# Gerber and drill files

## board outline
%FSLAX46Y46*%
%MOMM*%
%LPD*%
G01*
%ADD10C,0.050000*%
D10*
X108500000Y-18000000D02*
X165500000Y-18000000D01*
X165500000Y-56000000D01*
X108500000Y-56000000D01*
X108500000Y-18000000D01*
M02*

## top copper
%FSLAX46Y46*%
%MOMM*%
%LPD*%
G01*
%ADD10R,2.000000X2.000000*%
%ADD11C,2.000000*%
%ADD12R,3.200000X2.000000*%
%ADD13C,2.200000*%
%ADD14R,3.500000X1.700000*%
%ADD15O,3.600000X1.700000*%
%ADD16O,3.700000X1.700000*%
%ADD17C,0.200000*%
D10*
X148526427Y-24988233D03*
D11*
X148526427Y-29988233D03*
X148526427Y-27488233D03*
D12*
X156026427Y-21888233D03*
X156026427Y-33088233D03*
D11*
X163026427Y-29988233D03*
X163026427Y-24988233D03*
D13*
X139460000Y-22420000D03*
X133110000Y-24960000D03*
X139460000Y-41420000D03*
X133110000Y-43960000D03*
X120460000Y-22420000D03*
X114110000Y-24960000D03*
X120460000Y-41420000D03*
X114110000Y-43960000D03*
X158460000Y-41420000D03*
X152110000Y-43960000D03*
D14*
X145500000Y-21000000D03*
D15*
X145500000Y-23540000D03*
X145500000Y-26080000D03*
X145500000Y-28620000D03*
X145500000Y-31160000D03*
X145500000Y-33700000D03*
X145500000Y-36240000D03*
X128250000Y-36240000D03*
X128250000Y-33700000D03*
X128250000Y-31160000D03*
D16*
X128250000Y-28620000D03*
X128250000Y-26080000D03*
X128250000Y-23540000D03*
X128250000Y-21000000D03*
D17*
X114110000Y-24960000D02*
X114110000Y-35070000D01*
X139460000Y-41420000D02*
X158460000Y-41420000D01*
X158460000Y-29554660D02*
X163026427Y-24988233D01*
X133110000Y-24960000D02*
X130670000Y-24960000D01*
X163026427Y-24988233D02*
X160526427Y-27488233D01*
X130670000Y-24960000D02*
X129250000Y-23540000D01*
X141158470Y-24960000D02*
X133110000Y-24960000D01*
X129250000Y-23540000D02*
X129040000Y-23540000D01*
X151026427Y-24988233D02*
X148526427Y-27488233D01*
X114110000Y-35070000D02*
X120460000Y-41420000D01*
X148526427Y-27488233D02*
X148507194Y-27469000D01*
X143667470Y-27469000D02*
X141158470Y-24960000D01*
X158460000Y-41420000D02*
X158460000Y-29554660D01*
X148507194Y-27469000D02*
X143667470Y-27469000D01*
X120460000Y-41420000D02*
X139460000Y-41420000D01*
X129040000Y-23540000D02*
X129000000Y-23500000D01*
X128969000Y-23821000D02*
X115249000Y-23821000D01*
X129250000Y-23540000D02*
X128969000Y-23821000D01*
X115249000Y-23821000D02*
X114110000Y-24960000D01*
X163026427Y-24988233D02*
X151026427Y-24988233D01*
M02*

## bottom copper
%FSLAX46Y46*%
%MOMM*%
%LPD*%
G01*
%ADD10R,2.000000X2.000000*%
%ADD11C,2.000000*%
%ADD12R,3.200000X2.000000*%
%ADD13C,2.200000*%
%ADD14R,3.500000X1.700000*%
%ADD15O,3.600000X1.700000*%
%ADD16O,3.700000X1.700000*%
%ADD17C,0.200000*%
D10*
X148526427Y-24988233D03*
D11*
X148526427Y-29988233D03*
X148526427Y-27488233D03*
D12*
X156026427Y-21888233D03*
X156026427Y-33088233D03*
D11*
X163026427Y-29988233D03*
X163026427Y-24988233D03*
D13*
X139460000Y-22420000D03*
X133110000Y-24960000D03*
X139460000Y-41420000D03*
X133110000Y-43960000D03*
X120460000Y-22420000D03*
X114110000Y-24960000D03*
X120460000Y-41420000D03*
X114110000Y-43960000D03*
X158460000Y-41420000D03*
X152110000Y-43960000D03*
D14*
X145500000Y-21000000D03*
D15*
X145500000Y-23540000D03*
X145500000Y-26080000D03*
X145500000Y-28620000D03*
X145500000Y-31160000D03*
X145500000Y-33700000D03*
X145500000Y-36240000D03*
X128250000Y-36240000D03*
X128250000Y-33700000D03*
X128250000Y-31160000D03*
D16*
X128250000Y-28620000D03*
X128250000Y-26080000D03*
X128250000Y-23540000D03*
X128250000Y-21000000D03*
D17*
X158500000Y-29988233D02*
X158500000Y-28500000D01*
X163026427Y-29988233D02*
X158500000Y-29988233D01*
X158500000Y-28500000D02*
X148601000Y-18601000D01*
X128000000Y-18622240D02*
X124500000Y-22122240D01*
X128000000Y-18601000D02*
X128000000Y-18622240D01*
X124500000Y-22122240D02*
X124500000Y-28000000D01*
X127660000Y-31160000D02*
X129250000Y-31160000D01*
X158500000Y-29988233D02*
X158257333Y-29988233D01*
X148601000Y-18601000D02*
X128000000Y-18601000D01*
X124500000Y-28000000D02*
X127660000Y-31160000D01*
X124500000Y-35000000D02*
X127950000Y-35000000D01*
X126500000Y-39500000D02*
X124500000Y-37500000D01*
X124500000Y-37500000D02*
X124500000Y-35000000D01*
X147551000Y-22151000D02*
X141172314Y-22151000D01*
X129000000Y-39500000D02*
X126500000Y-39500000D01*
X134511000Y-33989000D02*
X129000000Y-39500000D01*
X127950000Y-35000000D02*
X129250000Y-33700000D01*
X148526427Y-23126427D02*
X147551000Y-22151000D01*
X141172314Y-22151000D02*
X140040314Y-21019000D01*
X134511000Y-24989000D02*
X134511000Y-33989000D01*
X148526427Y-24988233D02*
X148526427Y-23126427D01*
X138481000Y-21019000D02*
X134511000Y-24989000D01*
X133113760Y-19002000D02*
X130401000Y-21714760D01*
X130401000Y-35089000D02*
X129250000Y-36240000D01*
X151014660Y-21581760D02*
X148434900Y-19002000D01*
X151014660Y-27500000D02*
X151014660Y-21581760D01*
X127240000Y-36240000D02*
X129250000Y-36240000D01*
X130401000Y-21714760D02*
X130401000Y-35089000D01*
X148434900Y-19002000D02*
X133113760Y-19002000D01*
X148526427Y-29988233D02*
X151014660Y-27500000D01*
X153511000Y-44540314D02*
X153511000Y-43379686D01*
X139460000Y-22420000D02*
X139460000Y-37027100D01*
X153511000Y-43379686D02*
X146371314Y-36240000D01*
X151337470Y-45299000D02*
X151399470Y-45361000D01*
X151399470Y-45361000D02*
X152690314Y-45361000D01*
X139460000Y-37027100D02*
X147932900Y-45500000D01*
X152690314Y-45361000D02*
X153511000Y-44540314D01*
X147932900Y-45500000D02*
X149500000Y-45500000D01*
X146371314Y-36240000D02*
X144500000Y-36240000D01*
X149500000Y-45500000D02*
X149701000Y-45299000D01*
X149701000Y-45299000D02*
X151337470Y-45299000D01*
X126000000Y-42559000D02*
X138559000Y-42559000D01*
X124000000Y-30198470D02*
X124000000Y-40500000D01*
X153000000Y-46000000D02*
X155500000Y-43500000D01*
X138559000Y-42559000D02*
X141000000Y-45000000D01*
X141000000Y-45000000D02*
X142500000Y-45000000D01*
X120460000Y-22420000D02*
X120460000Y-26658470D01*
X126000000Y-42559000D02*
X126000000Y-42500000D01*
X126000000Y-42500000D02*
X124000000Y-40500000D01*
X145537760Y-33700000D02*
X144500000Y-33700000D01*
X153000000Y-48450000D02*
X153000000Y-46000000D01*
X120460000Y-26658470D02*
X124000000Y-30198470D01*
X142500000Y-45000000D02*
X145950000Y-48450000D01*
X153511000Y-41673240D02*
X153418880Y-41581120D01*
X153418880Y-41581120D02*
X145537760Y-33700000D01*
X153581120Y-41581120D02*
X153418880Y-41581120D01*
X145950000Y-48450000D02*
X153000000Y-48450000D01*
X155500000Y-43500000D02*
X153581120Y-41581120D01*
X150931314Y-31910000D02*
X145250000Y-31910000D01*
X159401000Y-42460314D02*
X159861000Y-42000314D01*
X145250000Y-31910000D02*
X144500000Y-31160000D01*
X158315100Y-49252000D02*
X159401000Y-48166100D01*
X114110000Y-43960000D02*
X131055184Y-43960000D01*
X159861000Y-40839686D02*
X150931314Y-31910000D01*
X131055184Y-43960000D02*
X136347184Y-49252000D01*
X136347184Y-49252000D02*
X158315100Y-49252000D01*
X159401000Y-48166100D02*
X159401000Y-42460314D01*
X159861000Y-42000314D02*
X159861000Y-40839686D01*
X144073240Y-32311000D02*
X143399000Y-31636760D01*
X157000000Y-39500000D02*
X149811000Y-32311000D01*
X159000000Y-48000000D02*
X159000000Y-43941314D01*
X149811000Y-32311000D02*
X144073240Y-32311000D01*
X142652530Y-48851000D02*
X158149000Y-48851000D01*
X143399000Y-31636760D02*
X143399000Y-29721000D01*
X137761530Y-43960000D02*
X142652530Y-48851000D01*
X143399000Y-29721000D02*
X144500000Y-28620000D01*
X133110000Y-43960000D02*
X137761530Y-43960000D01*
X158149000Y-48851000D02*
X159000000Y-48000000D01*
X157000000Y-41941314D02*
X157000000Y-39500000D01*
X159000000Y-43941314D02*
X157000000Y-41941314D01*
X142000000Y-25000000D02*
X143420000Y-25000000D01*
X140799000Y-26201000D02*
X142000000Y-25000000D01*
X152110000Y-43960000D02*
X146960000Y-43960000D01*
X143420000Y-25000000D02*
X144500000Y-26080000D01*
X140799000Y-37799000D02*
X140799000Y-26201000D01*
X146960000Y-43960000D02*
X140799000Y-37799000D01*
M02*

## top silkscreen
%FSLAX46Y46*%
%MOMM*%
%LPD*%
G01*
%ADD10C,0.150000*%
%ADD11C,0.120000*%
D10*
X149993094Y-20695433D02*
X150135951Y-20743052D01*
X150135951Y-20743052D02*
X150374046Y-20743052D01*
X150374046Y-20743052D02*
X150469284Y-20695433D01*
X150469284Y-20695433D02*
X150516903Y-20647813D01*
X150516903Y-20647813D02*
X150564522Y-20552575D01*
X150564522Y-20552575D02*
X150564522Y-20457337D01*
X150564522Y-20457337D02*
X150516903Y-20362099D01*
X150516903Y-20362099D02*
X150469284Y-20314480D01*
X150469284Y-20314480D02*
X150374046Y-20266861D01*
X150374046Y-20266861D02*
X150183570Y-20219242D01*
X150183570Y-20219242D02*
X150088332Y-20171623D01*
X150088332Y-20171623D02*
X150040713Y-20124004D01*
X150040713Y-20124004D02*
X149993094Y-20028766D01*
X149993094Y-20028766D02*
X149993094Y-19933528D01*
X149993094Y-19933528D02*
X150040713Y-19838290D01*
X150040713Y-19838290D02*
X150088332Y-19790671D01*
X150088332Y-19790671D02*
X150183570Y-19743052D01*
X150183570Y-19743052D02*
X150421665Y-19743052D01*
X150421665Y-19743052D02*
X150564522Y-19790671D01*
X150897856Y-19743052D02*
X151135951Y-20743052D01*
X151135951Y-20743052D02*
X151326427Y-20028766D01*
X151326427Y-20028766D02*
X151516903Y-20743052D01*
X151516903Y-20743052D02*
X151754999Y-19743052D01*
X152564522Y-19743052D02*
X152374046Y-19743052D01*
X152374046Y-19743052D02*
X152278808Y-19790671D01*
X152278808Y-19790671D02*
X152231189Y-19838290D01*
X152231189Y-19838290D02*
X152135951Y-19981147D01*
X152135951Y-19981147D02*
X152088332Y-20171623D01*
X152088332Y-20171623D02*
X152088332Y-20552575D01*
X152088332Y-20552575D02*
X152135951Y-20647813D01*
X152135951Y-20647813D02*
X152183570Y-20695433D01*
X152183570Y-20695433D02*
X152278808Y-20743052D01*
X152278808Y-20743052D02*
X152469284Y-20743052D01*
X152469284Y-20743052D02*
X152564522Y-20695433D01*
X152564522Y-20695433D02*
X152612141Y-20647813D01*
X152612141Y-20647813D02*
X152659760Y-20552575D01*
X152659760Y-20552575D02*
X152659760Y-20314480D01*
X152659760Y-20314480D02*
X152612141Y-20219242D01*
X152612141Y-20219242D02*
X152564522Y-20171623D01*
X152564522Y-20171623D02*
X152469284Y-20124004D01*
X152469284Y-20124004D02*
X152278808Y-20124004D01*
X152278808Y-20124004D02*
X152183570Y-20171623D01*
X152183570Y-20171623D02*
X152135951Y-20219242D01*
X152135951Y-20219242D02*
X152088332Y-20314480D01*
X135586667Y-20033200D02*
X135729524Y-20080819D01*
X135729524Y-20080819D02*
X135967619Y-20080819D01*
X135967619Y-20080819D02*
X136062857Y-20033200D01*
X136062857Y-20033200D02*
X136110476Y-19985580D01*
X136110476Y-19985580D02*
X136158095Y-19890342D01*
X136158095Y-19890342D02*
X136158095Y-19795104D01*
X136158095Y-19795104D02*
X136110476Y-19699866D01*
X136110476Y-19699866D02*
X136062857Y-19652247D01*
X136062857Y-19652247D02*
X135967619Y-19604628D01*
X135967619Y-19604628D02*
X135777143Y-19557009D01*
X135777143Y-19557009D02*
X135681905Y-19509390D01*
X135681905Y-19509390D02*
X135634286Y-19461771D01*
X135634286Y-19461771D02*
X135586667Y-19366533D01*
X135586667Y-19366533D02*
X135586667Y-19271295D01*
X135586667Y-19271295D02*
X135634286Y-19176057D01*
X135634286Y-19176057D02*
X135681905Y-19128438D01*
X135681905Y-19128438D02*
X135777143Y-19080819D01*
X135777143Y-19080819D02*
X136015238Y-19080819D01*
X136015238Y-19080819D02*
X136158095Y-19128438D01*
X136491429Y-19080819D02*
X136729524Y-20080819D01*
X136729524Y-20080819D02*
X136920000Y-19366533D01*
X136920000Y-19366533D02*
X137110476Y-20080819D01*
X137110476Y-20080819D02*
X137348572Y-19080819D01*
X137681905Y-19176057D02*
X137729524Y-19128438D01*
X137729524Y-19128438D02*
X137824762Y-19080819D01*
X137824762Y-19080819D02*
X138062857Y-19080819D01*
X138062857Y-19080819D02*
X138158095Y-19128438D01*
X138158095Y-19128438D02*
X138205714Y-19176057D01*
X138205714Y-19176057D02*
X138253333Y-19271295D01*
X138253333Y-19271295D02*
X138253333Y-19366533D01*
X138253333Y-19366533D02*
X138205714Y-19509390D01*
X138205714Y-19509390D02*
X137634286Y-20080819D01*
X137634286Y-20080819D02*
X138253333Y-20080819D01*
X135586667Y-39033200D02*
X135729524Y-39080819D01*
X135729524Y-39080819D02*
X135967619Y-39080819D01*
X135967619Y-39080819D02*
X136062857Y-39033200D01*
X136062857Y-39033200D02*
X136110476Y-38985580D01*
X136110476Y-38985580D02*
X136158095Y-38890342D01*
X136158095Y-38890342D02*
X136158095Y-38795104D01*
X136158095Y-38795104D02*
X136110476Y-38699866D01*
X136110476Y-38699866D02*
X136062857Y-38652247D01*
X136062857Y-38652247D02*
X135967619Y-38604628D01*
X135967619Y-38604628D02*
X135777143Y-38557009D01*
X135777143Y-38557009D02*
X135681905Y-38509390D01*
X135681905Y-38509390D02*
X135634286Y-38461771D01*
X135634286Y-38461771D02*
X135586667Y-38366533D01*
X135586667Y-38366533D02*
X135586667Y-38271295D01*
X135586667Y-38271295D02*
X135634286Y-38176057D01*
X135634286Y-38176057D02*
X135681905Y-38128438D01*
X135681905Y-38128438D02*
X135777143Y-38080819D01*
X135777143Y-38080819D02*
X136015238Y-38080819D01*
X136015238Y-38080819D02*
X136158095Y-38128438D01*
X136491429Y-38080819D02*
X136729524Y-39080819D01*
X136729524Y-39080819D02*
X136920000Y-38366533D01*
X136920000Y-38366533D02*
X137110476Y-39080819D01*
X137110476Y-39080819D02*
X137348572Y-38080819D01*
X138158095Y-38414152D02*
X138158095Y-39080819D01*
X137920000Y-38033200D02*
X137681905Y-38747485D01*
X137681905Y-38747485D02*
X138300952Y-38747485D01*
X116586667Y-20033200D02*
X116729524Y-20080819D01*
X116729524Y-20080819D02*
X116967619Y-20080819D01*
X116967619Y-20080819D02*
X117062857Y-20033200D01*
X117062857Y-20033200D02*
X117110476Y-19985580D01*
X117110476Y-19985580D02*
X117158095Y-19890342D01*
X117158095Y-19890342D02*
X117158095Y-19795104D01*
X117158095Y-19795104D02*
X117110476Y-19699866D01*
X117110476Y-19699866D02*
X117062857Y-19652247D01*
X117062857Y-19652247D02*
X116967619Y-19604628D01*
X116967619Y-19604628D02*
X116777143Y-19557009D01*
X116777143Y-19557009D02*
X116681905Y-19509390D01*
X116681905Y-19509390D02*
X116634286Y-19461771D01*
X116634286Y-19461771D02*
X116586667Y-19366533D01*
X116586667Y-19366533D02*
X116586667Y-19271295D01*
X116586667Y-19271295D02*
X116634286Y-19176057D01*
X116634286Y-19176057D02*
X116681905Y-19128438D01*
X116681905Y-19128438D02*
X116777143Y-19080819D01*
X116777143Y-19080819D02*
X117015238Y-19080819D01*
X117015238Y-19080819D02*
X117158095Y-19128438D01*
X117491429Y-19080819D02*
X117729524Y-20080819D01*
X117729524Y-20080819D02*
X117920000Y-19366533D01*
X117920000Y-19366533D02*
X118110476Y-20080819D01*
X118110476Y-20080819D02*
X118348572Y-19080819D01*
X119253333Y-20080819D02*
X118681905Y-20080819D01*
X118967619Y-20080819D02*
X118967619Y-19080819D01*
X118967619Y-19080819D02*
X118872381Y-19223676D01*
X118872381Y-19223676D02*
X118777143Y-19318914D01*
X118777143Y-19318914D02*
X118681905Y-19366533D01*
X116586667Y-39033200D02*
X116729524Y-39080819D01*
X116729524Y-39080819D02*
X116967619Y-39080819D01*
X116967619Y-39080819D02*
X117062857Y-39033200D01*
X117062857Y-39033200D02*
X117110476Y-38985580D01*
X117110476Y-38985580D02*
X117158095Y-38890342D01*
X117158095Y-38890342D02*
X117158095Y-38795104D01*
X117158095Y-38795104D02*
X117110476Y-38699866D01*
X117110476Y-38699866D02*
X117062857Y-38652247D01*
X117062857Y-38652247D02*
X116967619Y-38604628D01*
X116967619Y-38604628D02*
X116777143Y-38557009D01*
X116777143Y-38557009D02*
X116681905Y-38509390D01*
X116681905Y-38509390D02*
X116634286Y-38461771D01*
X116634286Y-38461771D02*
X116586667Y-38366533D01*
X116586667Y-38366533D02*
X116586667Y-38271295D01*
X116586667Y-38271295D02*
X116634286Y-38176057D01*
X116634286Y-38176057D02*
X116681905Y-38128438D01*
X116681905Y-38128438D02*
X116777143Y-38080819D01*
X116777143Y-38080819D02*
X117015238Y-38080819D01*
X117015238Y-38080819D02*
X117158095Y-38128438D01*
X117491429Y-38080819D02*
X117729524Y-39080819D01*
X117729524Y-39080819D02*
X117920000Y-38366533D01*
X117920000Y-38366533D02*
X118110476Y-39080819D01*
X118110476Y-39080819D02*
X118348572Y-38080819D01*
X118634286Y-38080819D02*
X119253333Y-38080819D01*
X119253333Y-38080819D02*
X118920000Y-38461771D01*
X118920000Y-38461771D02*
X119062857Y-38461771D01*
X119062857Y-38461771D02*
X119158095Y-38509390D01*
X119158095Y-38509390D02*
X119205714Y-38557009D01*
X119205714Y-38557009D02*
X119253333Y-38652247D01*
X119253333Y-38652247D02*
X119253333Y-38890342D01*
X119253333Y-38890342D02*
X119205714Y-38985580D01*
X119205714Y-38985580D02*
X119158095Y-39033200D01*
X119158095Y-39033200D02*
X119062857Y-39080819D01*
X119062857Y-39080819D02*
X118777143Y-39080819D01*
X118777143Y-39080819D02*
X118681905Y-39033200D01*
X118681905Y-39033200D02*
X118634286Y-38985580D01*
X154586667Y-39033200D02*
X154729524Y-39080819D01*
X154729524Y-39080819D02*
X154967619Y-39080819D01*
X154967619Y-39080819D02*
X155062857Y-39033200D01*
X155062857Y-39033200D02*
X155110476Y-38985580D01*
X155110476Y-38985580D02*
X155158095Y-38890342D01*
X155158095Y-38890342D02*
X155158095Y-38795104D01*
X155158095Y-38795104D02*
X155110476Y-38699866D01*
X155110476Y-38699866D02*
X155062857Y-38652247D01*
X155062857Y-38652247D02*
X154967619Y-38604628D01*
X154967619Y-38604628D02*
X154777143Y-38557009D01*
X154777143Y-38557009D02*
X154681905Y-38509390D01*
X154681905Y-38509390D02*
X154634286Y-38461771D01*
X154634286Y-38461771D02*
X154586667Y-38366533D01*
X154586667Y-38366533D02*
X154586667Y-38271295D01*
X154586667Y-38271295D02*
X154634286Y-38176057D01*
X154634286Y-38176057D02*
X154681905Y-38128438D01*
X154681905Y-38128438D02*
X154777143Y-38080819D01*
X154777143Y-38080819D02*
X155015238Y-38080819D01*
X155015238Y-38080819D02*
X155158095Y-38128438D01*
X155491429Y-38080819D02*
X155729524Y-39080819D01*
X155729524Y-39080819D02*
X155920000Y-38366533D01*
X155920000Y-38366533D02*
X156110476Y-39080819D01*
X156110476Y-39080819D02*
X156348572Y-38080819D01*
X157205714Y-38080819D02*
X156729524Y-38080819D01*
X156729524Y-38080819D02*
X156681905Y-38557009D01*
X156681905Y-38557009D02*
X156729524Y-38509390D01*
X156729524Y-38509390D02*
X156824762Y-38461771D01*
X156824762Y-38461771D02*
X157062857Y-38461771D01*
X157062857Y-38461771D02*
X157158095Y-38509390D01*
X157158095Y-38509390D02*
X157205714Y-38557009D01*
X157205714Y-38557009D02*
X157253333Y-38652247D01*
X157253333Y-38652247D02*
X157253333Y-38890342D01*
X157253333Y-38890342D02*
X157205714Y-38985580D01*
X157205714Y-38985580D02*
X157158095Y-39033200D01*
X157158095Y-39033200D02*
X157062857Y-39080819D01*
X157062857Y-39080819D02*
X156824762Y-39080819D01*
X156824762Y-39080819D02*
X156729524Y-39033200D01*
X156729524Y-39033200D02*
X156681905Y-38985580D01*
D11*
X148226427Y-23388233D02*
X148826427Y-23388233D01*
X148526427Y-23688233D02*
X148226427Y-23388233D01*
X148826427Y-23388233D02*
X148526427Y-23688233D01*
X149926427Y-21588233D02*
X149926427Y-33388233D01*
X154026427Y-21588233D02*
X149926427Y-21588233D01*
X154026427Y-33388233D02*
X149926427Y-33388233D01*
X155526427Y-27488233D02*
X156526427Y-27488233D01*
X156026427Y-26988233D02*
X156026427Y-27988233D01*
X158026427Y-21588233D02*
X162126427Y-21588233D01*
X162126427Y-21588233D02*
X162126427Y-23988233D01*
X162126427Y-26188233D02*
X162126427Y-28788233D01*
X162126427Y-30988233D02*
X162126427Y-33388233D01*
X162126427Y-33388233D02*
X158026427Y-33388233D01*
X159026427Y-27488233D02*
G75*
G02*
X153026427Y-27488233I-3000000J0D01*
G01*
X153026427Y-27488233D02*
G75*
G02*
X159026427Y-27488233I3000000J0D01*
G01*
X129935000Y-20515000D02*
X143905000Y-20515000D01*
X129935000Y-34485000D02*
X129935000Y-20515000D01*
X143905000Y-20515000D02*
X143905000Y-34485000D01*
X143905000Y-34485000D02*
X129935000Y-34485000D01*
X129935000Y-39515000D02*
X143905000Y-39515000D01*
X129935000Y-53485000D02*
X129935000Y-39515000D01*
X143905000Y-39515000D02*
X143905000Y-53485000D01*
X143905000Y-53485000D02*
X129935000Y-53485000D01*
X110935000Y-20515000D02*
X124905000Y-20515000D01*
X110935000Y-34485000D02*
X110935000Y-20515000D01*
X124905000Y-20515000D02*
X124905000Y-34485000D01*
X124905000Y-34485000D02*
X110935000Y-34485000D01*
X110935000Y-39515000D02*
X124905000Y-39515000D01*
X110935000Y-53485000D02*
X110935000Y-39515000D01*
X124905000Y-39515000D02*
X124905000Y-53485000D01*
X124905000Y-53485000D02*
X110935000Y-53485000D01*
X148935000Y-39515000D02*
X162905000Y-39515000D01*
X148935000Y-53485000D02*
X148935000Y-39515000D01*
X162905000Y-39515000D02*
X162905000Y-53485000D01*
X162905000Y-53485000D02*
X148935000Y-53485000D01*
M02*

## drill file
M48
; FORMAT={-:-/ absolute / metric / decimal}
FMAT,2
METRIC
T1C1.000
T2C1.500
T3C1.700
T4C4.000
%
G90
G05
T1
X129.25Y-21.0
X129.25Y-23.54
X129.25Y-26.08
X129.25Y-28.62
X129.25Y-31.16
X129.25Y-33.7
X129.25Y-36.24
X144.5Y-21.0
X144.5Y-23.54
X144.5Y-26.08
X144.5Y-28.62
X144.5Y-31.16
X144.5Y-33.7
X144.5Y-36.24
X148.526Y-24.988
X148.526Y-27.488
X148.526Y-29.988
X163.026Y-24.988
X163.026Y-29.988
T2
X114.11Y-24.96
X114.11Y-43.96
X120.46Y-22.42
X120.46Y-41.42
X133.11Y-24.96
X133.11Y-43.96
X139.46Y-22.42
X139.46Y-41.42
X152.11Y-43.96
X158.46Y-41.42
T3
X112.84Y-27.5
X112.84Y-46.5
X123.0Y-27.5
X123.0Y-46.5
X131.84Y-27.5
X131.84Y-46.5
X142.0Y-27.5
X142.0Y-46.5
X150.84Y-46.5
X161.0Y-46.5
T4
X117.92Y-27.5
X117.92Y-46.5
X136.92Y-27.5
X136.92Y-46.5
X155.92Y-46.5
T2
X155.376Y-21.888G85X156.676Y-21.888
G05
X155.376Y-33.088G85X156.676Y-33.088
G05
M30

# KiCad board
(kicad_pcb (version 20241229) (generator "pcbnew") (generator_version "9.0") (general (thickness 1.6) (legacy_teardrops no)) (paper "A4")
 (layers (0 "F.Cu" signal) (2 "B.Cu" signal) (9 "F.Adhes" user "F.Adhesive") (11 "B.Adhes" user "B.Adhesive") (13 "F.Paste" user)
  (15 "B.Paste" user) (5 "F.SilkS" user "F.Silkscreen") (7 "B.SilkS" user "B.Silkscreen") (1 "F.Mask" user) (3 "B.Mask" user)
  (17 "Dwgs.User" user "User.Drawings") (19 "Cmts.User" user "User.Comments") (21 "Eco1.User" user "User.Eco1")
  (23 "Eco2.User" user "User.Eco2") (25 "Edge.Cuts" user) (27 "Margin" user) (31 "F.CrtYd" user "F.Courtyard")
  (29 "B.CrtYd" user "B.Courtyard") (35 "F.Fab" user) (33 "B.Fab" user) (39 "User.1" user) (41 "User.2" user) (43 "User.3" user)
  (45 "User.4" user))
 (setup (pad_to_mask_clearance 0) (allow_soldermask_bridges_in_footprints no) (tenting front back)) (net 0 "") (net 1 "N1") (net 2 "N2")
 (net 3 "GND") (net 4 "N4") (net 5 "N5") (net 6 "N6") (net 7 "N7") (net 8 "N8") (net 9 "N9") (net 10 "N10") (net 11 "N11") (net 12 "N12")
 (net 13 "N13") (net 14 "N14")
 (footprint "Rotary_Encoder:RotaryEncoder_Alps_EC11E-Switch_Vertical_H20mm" (layer "F.Cu") (at 148.526427 24.988233)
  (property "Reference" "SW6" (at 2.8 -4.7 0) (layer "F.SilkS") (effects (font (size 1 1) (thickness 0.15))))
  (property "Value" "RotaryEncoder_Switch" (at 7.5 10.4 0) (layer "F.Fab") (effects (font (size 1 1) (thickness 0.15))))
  (fp_line (start -0.3 -1.6) (end 0.3 -1.6) (stroke (width 0.12) (type solid)) (layer "F.SilkS"))
  (fp_line (start 0 -1.3) (end -0.3 -1.6) (stroke (width 0.12) (type solid)) (layer "F.SilkS"))
  (fp_line (start 0.3 -1.6) (end 0 -1.3) (stroke (width 0.12) (type solid)) (layer "F.SilkS"))
  (fp_line (start 1.4 -3.4) (end 1.4 8.4) (stroke (width 0.12) (type solid)) (layer "F.SilkS"))
  (fp_line (start 5.5 -3.4) (end 1.4 -3.4) (stroke (width 0.12) (type solid)) (layer "F.SilkS"))
  (fp_line (start 5.5 8.4) (end 1.4 8.4) (stroke (width 0.12) (type solid)) (layer "F.SilkS"))
  (fp_line (start 7 2.5) (end 8 2.5) (stroke (width 0.12) (type solid)) (layer "F.SilkS"))
  (fp_line (start 7.5 2) (end 7.5 3) (stroke (width 0.12) (type solid)) (layer "F.SilkS"))
  (fp_line (start 9.5 -3.4) (end 13.6 -3.4) (stroke (width 0.12) (type solid)) (layer "F.SilkS"))
  (fp_line (start 13.6 -3.4) (end 13.6 -1) (stroke (width 0.12) (type solid)) (layer "F.SilkS"))
  (fp_line (start 13.6 1.2) (end 13.6 3.8) (stroke (width 0.12) (type solid)) (layer "F.SilkS"))
  (fp_line (start 13.6 6) (end 13.6 8.4) (stroke (width 0.12) (type solid)) (layer "F.SilkS"))
  (fp_line (start 13.6 8.4) (end 9.5 8.4) (stroke (width 0.12) (type solid)) (layer "F.SilkS"))
  (fp_circle (center 7.5 2.5) (end 10.5 2.5) (stroke (width 0.12) (type solid)) (fill no) (layer "F.SilkS"))
  (pad "A" thru_hole rect (at 0 0) (size 2 2) (drill 1) (layers "*.Cu" "*.Mask") (remove_unused_layers no) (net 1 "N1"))
  (pad "B" thru_hole circle (at 0 5) (size 2 2) (drill 1) (layers "*.Cu" "*.Mask") (remove_unused_layers no) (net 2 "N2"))
  (pad "C" thru_hole circle (at 0 2.5) (size 2 2) (drill 1) (layers "*.Cu" "*.Mask") (remove_unused_layers no) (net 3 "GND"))
  (pad "MP" thru_hole rect (at 7.5 -3.1) (size 3.2 2) (drill oval 2.8 1.5) (layers "*.Cu" "*.Mask") (remove_unused_layers no))
  (pad "MP" thru_hole rect (at 7.5 8.1) (size 3.2 2) (drill oval 2.8 1.5) (layers "*.Cu" "*.Mask") (remove_unused_layers no))
  (pad "S1" thru_hole circle (at 14.5 5) (size 2 2) (drill 1) (layers "*.Cu" "*.Mask") (remove_unused_layers no) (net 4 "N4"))
  (pad "S2" thru_hole circle (at 14.5 0) (size 2 2) (drill 1) (layers "*.Cu" "*.Mask") (remove_unused_layers no) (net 3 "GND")))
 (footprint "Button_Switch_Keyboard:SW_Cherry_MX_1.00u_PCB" (layer "F.Cu") (at 139.46 22.42)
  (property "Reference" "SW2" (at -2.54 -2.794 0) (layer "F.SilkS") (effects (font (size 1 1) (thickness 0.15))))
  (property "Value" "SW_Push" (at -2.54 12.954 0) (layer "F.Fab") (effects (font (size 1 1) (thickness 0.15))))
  (fp_line (start -9.525 -1.905) (end 4.445 -1.905) (stroke (width 0.12) (type solid)) (layer "F.SilkS"))
  (fp_line (start -9.525 12.065) (end -9.525 -1.905) (stroke (width 0.12) (type solid)) (layer "F.SilkS"))
  (fp_line (start 4.445 -1.905) (end 4.445 12.065) (stroke (width 0.12) (type solid)) (layer "F.SilkS"))
  (fp_line (start 4.445 12.065) (end -9.525 12.065) (stroke (width 0.12) (type solid)) (layer "F.SilkS"))
  (pad "" np_thru_hole circle (at -7.62 5.08) (size 1.7 1.7) (drill 1.7) (layers "*.Cu" "*.Mask"))
  (pad "" np_thru_hole circle (at -2.54 5.08) (size 4 4) (drill 4) (layers "*.Cu" "*.Mask"))
  (pad "" np_thru_hole circle (at 2.54 5.08) (size 1.7 1.7) (drill 1.7) (layers "*.Cu" "*.Mask"))
  (pad "1" thru_hole circle (at 0 0) (size 2.2 2.2) (drill 1.5) (layers "*.Cu" "*.Mask") (remove_unused_layers no) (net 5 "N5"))
  (pad "2" thru_hole circle (at -6.35 2.54) (size 2.2 2.2) (drill 1.5) (layers "*.Cu" "*.Mask") (remove_unused_layers no) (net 3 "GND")))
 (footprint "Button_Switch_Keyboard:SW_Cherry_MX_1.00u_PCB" (layer "F.Cu") (at 139.46 41.42)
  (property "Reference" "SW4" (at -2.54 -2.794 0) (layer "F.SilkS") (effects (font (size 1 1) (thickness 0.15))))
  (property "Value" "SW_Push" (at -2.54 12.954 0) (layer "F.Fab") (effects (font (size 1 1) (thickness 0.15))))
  (fp_line (start -9.525 -1.905) (end 4.445 -1.905) (stroke (width 0.12) (type solid)) (layer "F.SilkS"))
  (fp_line (start -9.525 12.065) (end -9.525 -1.905) (stroke (width 0.12) (type solid)) (layer "F.SilkS"))
  (fp_line (start 4.445 -1.905) (end 4.445 12.065) (stroke (width 0.12) (type solid)) (layer "F.SilkS"))
  (fp_line (start 4.445 12.065) (end -9.525 12.065) (stroke (width 0.12) (type solid)) (layer "F.SilkS"))
  (pad "" np_thru_hole circle (at -7.62 5.08) (size 1.7 1.7) (drill 1.7) (layers "*.Cu" "*.Mask"))
  (pad "" np_thru_hole circle (at -2.54 5.08) (size 4 4) (drill 4) (layers "*.Cu" "*.Mask"))
  (pad "" np_thru_hole circle (at 2.54 5.08) (size 1.7 1.7) (drill 1.7) (layers "*.Cu" "*.Mask"))
  (pad "1" thru_hole circle (at 0 0) (size 2.2 2.2) (drill 1.5) (layers "*.Cu" "*.Mask") (remove_unused_layers no) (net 3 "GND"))
  (pad "2" thru_hole circle (at -6.35 2.54) (size 2.2 2.2) (drill 1.5) (layers "*.Cu" "*.Mask") (remove_unused_layers no) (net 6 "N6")))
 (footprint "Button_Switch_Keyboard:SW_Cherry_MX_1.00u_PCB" (layer "F.Cu") (at 120.46 22.42)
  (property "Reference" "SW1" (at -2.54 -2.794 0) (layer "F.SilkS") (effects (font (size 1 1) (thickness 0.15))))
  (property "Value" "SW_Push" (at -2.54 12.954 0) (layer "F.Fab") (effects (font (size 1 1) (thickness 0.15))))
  (fp_line (start -9.525 -1.905) (end 4.445 -1.905) (stroke (width 0.12) (type solid)) (layer "F.SilkS"))
  (fp_line (start -9.525 12.065) (end -9.525 -1.905) (stroke (width 0.12) (type solid)) (layer "F.SilkS"))
  (fp_line (start 4.445 -1.905) (end 4.445 12.065) (stroke (width 0.12) (type solid)) (layer "F.SilkS"))
  (fp_line (start 4.445 12.065) (end -9.525 12.065) (stroke (width 0.12) (type solid)) (layer "F.SilkS"))
  (pad "" np_thru_hole circle (at -7.62 5.08) (size 1.7 1.7) (drill 1.7) (layers "*.Cu" "*.Mask"))
  (pad "" np_thru_hole circle (at -2.54 5.08) (size 4 4) (drill 4) (layers "*.Cu" "*.Mask"))
  (pad "" np_thru_hole circle (at 2.54 5.08) (size 1.7 1.7) (drill 1.7) (layers "*.Cu" "*.Mask"))
  (pad "1" thru_hole circle (at 0 0) (size 2.2 2.2) (drill 1.5) (layers "*.Cu" "*.Mask") (remove_unused_layers no) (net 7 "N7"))
  (pad "2" thru_hole circle (at -6.35 2.54) (size 2.2 2.2) (drill 1.5) (layers "*.Cu" "*.Mask") (remove_unused_layers no) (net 3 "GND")))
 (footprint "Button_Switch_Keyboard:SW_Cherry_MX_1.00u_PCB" (layer "F.Cu") (at 120.46 41.42)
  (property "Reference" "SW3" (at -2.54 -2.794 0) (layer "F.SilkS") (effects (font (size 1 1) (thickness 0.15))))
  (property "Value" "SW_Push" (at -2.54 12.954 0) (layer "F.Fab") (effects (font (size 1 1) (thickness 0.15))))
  (fp_line (start -9.525 -1.905) (end 4.445 -1.905) (stroke (width 0.12) (type solid)) (layer "F.SilkS"))
  (fp_line (start -9.525 12.065) (end -9.525 -1.905) (stroke (width 0.12) (type solid)) (layer "F.SilkS"))
  (fp_line (start 4.445 -1.905) (end 4.445 12.065) (stroke (width 0.12) (type solid)) (layer "F.SilkS"))
  (fp_line (start 4.445 12.065) (end -9.525 12.065) (stroke (width 0.12) (type solid)) (layer "F.SilkS"))
  (pad "" np_thru_hole circle (at -7.62 5.08) (size 1.7 1.7) (drill 1.7) (layers "*.Cu" "*.Mask"))
  (pad "" np_thru_hole circle (at -2.54 5.08) (size 4 4) (drill 4) (layers "*.Cu" "*.Mask"))
  (pad "" np_thru_hole circle (at 2.54 5.08) (size 1.7 1.7) (drill 1.7) (layers "*.Cu" "*.Mask"))
  (pad "1" thru_hole circle (at 0 0) (size 2.2 2.2) (drill 1.5) (layers "*.Cu" "*.Mask") (remove_unused_layers no) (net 3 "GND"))
  (pad "2" thru_hole circle (at -6.35 2.54) (size 2.2 2.2) (drill 1.5) (layers "*.Cu" "*.Mask") (remove_unused_layers no) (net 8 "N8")))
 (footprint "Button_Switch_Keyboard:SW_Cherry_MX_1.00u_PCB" (layer "F.Cu") (at 158.46 41.42)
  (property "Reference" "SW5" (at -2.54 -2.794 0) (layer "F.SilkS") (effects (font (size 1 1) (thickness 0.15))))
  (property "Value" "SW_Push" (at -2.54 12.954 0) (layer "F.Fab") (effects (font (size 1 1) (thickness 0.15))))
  (fp_line (start -9.525 -1.905) (end 4.445 -1.905) (stroke (width 0.12) (type solid)) (layer "F.SilkS"))
  (fp_line (start -9.525 12.065) (end -9.525 -1.905) (stroke (width 0.12) (type solid)) (layer "F.SilkS"))
  (fp_line (start 4.445 -1.905) (end 4.445 12.065) (stroke (width 0.12) (type solid)) (layer "F.SilkS"))
  (fp_line (start 4.445 12.065) (end -9.525 12.065) (stroke (width 0.12) (type solid)) (layer "F.SilkS"))
  (pad "" np_thru_hole circle (at -7.62 5.08) (size 1.7 1.7) (drill 1.7) (layers "*.Cu" "*.Mask"))
  (pad "" np_thru_hole circle (at -2.54 5.08) (size 4 4) (drill 4) (layers "*.Cu" "*.Mask"))
  (pad "" np_thru_hole circle (at 2.54 5.08) (size 1.7 1.7) (drill 1.7) (layers "*.Cu" "*.Mask"))
  (pad "1" thru_hole circle (at 0 0) (size 2.2 2.2) (drill 1.5) (layers "*.Cu" "*.Mask") (remove_unused_layers no) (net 3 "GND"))
  (pad "2" thru_hole circle (at -6.35 2.54) (size 2.2 2.2) (drill 1.5) (layers "*.Cu" "*.Mask") (remove_unused_layers no) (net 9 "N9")))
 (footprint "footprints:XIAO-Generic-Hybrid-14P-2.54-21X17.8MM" (layer "B.Cu") (at 136.875 28.62 180)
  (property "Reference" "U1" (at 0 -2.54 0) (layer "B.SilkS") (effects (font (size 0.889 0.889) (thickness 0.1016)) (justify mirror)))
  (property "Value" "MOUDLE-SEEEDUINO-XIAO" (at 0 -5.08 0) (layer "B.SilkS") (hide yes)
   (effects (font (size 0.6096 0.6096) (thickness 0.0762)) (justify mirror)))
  (pad "1" thru_hole rect (at -7.625 7.62 180) (size 3.5 1.7) (drill 1 (offset -1 0)) (layers "*.Cu" "*.Mask") (remove_unused_layers no)
   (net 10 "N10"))
  (pad "2" thru_hole oval (at -7.625 5.08 180) (size 3.6 1.7) (drill 1 (offset -1 0)) (layers "*.Cu" "*.Mask") (remove_unused_layers no)
   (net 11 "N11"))
  (pad "3" thru_hole oval (at -7.625 2.54 180) (size 3.6 1.7) (drill 1 (offset -1 0)) (layers "*.Cu" "*.Mask") (remove_unused_layers no)
   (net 9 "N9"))
  (pad "4" thru_hole oval (at -7.625 0 180) (size 3.6 1.7) (drill 1 (offset -1 0)) (layers "*.Cu" "*.Mask") (remove_unused_layers no)
   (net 6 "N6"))
  (pad "5" thru_hole oval (at -7.625 -2.54 180) (size 3.6 1.7) (drill 1 (offset -1 0)) (layers "*.Cu" "*.Mask") (remove_unused_layers no)
   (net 8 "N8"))
  (pad "6" thru_hole oval (at -7.625 -5.08) (size 3.6 1.7) (drill 1 (offset 1 0)) (layers "*.Cu" "*.Mask") (remove_unused_layers no)
   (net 7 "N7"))
  (pad "7" thru_hole oval (at -7.625 -7.62 180) (size 3.6 1.7) (drill 1 (offset -1 0)) (layers "*.Cu" "*.Mask") (remove_unused_layers no)
   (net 5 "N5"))
  (pad "8" thru_hole oval (at 7.625 -7.62 180) (size 3.6 1.7) (drill 1 (offset 1 0)) (layers "*.Cu" "*.Mask") (remove_unused_layers no)
   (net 2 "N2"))
  (pad "9" thru_hole oval (at 7.625 -5.08 180) (size 3.6 1.7) (drill 1 (offset 1 0)) (layers "*.Cu" "*.Mask") (remove_unused_layers no)
   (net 1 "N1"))
  (pad "10" thru_hole oval (at 7.625 -2.54 180) (size 3.6 1.7) (drill 1 (offset 1 0)) (layers "*.Cu" "*.Mask") (remove_unused_layers no)
   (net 4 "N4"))
  (pad "11" thru_hole oval (at 7.625 0 180) (size 3.7 1.7) (drill 1 (offset 1 0)) (layers "*.Cu" "*.Mask") (remove_unused_layers no)
   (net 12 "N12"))
  (pad "12" thru_hole oval (at 7.625 2.54 180) (size 3.7 1.7) (drill 1 (offset 1 0)) (layers "*.Cu" "*.Mask") (remove_unused_layers no)
   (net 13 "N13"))
  (pad "13" thru_hole oval (at 7.625 5.08 180) (size 3.7 1.7) (drill 1 (offset 1 0)) (layers "*.Cu" "*.Mask") (remove_unused_layers no)
   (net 3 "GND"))
  (pad "14" thru_hole oval (at 7.625 7.62 180) (size 3.7 1.7) (drill 1 (offset 1 0)) (layers "*.Cu" "*.Mask") (remove_unused_layers no)
   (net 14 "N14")))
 (gr_rect (start 108.5 18) (end 165.5 56) (stroke (width 0.05) (type default)) (fill no) (layer "Edge.Cuts"))
 (segment (start 114.11 24.96) (end 114.11 35.07) (width 0.2) (layer "F.Cu") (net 3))
 (segment (start 139.46 41.42) (end 158.46 41.42) (width 0.2) (layer "F.Cu") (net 3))
 (segment (start 158.46 29.55466) (end 163.026427 24.988233) (width 0.2) (layer "F.Cu") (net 3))
 (segment (start 133.11 24.96) (end 130.67 24.96) (width 0.2) (layer "F.Cu") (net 3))
 (segment (start 163.026427 24.988233) (end 160.526427 27.488233) (width 0.2) (layer "F.Cu") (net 3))
 (segment (start 130.67 24.96) (end 129.25 23.54) (width 0.2) (layer "F.Cu") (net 3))
 (segment (start 141.15847 24.96) (end 133.11 24.96) (width 0.2) (layer "F.Cu") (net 3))
 (segment (start 129.25 23.54) (end 129.04 23.54) (width 0.2) (layer "F.Cu") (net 3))
 (segment (start 151.026427 24.988233) (end 148.526427 27.488233) (width 0.2) (layer "F.Cu") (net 3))
 (segment (start 114.11 35.07) (end 120.46 41.42) (width 0.2) (layer "F.Cu") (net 3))
 (segment (start 148.526427 27.488233) (end 148.507194 27.469) (width 0.2) (layer "F.Cu") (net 3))
 (segment (start 143.66747 27.469) (end 141.15847 24.96) (width 0.2) (layer "F.Cu") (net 3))
 (segment (start 158.46 41.42) (end 158.46 29.55466) (width 0.2) (layer "F.Cu") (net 3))
 (segment (start 148.507194 27.469) (end 143.66747 27.469) (width 0.2) (layer "F.Cu") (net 3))
 (segment (start 120.46 41.42) (end 139.46 41.42) (width 0.2) (layer "F.Cu") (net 3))
 (segment (start 129.04 23.54) (end 129 23.5) (width 0.2) (layer "F.Cu") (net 3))
 (segment (start 128.969 23.821) (end 115.249 23.821) (width 0.2) (layer "F.Cu") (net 3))
 (segment (start 129.25 23.54) (end 128.969 23.821) (width 0.2) (layer "F.Cu") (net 3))
 (segment (start 115.249 23.821) (end 114.11 24.96) (width 0.2) (layer "F.Cu") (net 3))
 (segment (start 163.026427 24.988233) (end 151.026427 24.988233) (width 0.2) (layer "F.Cu") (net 3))
 (segment (start 158.5 29.988233) (end 158.5 28.5) (width 0.2) (layer "B.Cu") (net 4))
 (segment (start 163.026427 29.988233) (end 158.5 29.988233) (width 0.2) (layer "B.Cu") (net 4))
 (segment (start 158.5 28.5) (end 148.601 18.601) (width 0.2) (layer "B.Cu") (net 4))
 (segment (start 128 18.62224) (end 124.5 22.12224) (width 0.2) (layer "B.Cu") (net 4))
 (segment (start 128 18.601) (end 128 18.62224) (width 0.2) (layer "B.Cu") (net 4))
 (segment (start 124.5 22.12224) (end 124.5 28) (width 0.2) (layer "B.Cu") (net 4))
 (segment (start 127.66 31.16) (end 129.25 31.16) (width 0.2) (layer "B.Cu") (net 4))
 (segment (start 158.5 29.988233) (end 158.257333 29.988233) (width 0.2) (layer "B.Cu") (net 4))
 (segment (start 148.601 18.601) (end 128 18.601) (width 0.2) (layer "B.Cu") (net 4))
 (segment (start 124.5 28) (end 127.66 31.16) (width 0.2) (layer "B.Cu") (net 4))
 (segment (start 124.5 35) (end 127.95 35) (width 0.2) (layer "B.Cu") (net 1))
 (segment (start 126.5 39.5) (end 124.5 37.5) (width 0.2) (layer "B.Cu") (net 1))
 (segment (start 124.5 37.5) (end 124.5 35) (width 0.2) (layer "B.Cu") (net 1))
 (segment (start 147.551 22.151) (end 141.172314 22.151) (width 0.2) (layer "B.Cu") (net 1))
 (segment (start 129 39.5) (end 126.5 39.5) (width 0.2) (layer "B.Cu") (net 1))
 (segment (start 134.511 33.989) (end 129 39.5) (width 0.2) (layer "B.Cu") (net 1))
 (segment (start 127.95 35) (end 129.25 33.7) (width 0.2) (layer "B.Cu") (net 1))
 (segment (start 148.526427 23.126427) (end 147.551 22.151) (width 0.2) (layer "B.Cu") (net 1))
 (segment (start 141.172314 22.151) (end 140.040314 21.019) (width 0.2) (layer "B.Cu") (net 1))
 (segment (start 134.511 24.989) (end 134.511 33.989) (width 0.2) (layer "B.Cu") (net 1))
 (segment (start 148.526427 24.988233) (end 148.526427 23.126427) (width 0.2) (layer "B.Cu") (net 1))
 (segment (start 138.481 21.019) (end 134.511 24.989) (width 0.2) (layer "B.Cu") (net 1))
 (segment (start 133.11376 19.002) (end 130.401 21.71476) (width 0.2) (layer "B.Cu") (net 2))
 (segment (start 130.401 35.089) (end 129.25 36.24) (width 0.2) (layer "B.Cu") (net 2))
 (segment (start 151.01466 21.58176) (end 148.4349 19.002) (width 0.2) (layer "B.Cu") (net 2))
 (segment (start 151.01466 27.5) (end 151.01466 21.58176) (width 0.2) (layer "B.Cu") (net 2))
 (segment (start 127.24 36.24) (end 129.25 36.24) (width 0.2) (layer "B.Cu") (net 2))
 (segment (start 130.401 21.71476) (end 130.401 35.089) (width 0.2) (layer "B.Cu") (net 2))
 (segment (start 148.4349 19.002) (end 133.11376 19.002) (width 0.2) (layer "B.Cu") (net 2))
 (segment (start 148.526427 29.988233) (end 151.01466 27.5) (width 0.2) (layer "B.Cu") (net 2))
 (segment (start 153.511 44.540314) (end 153.511 43.379686) (width 0.2) (layer "B.Cu") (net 5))
 (segment (start 139.46 22.42) (end 139.46 37.0271) (width 0.2) (layer "B.Cu") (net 5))
 (segment (start 153.511 43.379686) (end 146.371314 36.24) (width 0.2) (layer "B.Cu") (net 5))
 (segment (start 151.33747 45.299) (end 151.39947 45.361) (width 0.2) (layer "B.Cu") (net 5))
 (segment (start 151.39947 45.361) (end 152.690314 45.361) (width 0.2) (layer "B.Cu") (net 5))
 (segment (start 139.46 37.0271) (end 147.9329 45.5) (width 0.2) (layer "B.Cu") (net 5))
 (segment (start 152.690314 45.361) (end 153.511 44.540314) (width 0.2) (layer "B.Cu") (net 5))
 (segment (start 147.9329 45.5) (end 149.5 45.5) (width 0.2) (layer "B.Cu") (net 5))
 (segment (start 146.371314 36.24) (end 144.5 36.24) (width 0.2) (layer "B.Cu") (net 5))
 (segment (start 149.5 45.5) (end 149.701 45.299) (width 0.2) (layer "B.Cu") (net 5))
 (segment (start 149.701 45.299) (end 151.33747 45.299) (width 0.2) (layer "B.Cu") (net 5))
 (segment (start 126 42.559) (end 138.559 42.559) (width 0.2) (layer "B.Cu") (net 7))
 (segment (start 124 30.19847) (end 124 40.5) (width 0.2) (layer "B.Cu") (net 7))
 (segment (start 153 46) (end 155.5 43.5) (width 0.2) (layer "B.Cu") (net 7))
 (segment (start 138.559 42.559) (end 141 45) (width 0.2) (layer "B.Cu") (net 7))
 (segment (start 141 45) (end 142.5 45) (width 0.2) (layer "B.Cu") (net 7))
 (segment (start 120.46 22.42) (end 120.46 26.65847) (width 0.2) (layer "B.Cu") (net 7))
 (segment (start 126 42.559) (end 126 42.5) (width 0.2) (layer "B.Cu") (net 7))
 (segment (start 126 42.5) (end 124 40.5) (width 0.2) (layer "B.Cu") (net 7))
 (segment (start 145.53776 33.7) (end 144.5 33.7) (width 0.2) (layer "B.Cu") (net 7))
 (segment (start 153 48.45) (end 153 46) (width 0.2) (layer "B.Cu") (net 7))
 (segment (start 120.46 26.65847) (end 124 30.19847) (width 0.2) (layer "B.Cu") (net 7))
 (segment (start 142.5 45) (end 145.95 48.45) (width 0.2) (layer "B.Cu") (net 7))
 (segment (start 153.511 41.67324) (end 153.41888 41.58112) (width 0.2) (layer "B.Cu") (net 7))
 (segment (start 153.41888 41.58112) (end 145.53776 33.7) (width 0.2) (layer "B.Cu") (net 7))
 (segment (start 153.58112 41.58112) (end 153.41888 41.58112) (width 0.2) (layer "B.Cu") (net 7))
 (segment (start 145.95 48.45) (end 153 48.45) (width 0.2) (layer "B.Cu") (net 7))
 (segment (start 155.5 43.5) (end 153.58112 41.58112) (width 0.2) (layer "B.Cu") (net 7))
 (segment (start 150.931314 31.91) (end 145.25 31.91) (width 0.2) (layer "B.Cu") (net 8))
 (segment (start 159.401 42.460314) (end 159.861 42.000314) (width 0.2) (layer "B.Cu") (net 8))
 (segment (start 145.25 31.91) (end 144.5 31.16) (width 0.2) (layer "B.Cu") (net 8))
 (segment (start 158.3151 49.252) (end 159.401 48.1661) (width 0.2) (layer "B.Cu") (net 8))
 (segment (start 114.11 43.96) (end 131.055184 43.96) (width 0.2) (layer "B.Cu") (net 8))
 (segment (start 159.861 40.839686) (end 150.931314 31.91) (width 0.2) (layer "B.Cu") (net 8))
 (segment (start 131.055184 43.96) (end 136.347184 49.252) (width 0.2) (layer "B.Cu") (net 8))
 (segment (start 136.347184 49.252) (end 158.3151 49.252) (width 0.2) (layer "B.Cu") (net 8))
 (segment (start 159.401 48.1661) (end 159.401 42.460314) (width 0.2) (layer "B.Cu") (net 8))
 (segment (start 159.861 42.000314) (end 159.861 40.839686) (width 0.2) (layer "B.Cu") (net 8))
 (segment (start 144.07324 32.311) (end 143.399 31.63676) (width 0.2) (layer "B.Cu") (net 6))
 (segment (start 157 39.5) (end 149.811 32.311) (width 0.2) (layer "B.Cu") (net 6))
 (segment (start 159 48) (end 159 43.941314) (width 0.2) (layer "B.Cu") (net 6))
 (segment (start 149.811 32.311) (end 144.07324 32.311) (width 0.2) (layer "B.Cu") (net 6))
 (segment (start 142.65253 48.851) (end 158.149 48.851) (width 0.2) (layer "B.Cu") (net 6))
 (segment (start 143.399 31.63676) (end 143.399 29.721) (width 0.2) (layer "B.Cu") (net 6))
 (segment (start 137.76153 43.96) (end 142.65253 48.851) (width 0.2) (layer "B.Cu") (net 6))
 (segment (start 143.399 29.721) (end 144.5 28.62) (width 0.2) (layer "B.Cu") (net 6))
 (segment (start 133.11 43.96) (end 137.76153 43.96) (width 0.2) (layer "B.Cu") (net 6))
 (segment (start 158.149 48.851) (end 159 48) (width 0.2) (layer "B.Cu") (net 6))
 (segment (start 157 41.941314) (end 157 39.5) (width 0.2) (layer "B.Cu") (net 6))
 (segment (start 159 43.941314) (end 157 41.941314) (width 0.2) (layer "B.Cu") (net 6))
 (segment (start 142 25) (end 143.42 25) (width 0.2) (layer "B.Cu") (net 9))
 (segment (start 140.799 26.201) (end 142 25) (width 0.2) (layer "B.Cu") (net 9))
 (segment (start 152.11 43.96) (end 146.96 43.96) (width 0.2) (layer "B.Cu") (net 9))
 (segment (start 143.42 25) (end 144.5 26.08) (width 0.2) (layer "B.Cu") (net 9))
 (segment (start 140.799 37.799) (end 140.799 26.201) (width 0.2) (layer "B.Cu") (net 9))
 (segment (start 146.96 43.96) (end 140.799 37.799) (width 0.2) (layer "B.Cu") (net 9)))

